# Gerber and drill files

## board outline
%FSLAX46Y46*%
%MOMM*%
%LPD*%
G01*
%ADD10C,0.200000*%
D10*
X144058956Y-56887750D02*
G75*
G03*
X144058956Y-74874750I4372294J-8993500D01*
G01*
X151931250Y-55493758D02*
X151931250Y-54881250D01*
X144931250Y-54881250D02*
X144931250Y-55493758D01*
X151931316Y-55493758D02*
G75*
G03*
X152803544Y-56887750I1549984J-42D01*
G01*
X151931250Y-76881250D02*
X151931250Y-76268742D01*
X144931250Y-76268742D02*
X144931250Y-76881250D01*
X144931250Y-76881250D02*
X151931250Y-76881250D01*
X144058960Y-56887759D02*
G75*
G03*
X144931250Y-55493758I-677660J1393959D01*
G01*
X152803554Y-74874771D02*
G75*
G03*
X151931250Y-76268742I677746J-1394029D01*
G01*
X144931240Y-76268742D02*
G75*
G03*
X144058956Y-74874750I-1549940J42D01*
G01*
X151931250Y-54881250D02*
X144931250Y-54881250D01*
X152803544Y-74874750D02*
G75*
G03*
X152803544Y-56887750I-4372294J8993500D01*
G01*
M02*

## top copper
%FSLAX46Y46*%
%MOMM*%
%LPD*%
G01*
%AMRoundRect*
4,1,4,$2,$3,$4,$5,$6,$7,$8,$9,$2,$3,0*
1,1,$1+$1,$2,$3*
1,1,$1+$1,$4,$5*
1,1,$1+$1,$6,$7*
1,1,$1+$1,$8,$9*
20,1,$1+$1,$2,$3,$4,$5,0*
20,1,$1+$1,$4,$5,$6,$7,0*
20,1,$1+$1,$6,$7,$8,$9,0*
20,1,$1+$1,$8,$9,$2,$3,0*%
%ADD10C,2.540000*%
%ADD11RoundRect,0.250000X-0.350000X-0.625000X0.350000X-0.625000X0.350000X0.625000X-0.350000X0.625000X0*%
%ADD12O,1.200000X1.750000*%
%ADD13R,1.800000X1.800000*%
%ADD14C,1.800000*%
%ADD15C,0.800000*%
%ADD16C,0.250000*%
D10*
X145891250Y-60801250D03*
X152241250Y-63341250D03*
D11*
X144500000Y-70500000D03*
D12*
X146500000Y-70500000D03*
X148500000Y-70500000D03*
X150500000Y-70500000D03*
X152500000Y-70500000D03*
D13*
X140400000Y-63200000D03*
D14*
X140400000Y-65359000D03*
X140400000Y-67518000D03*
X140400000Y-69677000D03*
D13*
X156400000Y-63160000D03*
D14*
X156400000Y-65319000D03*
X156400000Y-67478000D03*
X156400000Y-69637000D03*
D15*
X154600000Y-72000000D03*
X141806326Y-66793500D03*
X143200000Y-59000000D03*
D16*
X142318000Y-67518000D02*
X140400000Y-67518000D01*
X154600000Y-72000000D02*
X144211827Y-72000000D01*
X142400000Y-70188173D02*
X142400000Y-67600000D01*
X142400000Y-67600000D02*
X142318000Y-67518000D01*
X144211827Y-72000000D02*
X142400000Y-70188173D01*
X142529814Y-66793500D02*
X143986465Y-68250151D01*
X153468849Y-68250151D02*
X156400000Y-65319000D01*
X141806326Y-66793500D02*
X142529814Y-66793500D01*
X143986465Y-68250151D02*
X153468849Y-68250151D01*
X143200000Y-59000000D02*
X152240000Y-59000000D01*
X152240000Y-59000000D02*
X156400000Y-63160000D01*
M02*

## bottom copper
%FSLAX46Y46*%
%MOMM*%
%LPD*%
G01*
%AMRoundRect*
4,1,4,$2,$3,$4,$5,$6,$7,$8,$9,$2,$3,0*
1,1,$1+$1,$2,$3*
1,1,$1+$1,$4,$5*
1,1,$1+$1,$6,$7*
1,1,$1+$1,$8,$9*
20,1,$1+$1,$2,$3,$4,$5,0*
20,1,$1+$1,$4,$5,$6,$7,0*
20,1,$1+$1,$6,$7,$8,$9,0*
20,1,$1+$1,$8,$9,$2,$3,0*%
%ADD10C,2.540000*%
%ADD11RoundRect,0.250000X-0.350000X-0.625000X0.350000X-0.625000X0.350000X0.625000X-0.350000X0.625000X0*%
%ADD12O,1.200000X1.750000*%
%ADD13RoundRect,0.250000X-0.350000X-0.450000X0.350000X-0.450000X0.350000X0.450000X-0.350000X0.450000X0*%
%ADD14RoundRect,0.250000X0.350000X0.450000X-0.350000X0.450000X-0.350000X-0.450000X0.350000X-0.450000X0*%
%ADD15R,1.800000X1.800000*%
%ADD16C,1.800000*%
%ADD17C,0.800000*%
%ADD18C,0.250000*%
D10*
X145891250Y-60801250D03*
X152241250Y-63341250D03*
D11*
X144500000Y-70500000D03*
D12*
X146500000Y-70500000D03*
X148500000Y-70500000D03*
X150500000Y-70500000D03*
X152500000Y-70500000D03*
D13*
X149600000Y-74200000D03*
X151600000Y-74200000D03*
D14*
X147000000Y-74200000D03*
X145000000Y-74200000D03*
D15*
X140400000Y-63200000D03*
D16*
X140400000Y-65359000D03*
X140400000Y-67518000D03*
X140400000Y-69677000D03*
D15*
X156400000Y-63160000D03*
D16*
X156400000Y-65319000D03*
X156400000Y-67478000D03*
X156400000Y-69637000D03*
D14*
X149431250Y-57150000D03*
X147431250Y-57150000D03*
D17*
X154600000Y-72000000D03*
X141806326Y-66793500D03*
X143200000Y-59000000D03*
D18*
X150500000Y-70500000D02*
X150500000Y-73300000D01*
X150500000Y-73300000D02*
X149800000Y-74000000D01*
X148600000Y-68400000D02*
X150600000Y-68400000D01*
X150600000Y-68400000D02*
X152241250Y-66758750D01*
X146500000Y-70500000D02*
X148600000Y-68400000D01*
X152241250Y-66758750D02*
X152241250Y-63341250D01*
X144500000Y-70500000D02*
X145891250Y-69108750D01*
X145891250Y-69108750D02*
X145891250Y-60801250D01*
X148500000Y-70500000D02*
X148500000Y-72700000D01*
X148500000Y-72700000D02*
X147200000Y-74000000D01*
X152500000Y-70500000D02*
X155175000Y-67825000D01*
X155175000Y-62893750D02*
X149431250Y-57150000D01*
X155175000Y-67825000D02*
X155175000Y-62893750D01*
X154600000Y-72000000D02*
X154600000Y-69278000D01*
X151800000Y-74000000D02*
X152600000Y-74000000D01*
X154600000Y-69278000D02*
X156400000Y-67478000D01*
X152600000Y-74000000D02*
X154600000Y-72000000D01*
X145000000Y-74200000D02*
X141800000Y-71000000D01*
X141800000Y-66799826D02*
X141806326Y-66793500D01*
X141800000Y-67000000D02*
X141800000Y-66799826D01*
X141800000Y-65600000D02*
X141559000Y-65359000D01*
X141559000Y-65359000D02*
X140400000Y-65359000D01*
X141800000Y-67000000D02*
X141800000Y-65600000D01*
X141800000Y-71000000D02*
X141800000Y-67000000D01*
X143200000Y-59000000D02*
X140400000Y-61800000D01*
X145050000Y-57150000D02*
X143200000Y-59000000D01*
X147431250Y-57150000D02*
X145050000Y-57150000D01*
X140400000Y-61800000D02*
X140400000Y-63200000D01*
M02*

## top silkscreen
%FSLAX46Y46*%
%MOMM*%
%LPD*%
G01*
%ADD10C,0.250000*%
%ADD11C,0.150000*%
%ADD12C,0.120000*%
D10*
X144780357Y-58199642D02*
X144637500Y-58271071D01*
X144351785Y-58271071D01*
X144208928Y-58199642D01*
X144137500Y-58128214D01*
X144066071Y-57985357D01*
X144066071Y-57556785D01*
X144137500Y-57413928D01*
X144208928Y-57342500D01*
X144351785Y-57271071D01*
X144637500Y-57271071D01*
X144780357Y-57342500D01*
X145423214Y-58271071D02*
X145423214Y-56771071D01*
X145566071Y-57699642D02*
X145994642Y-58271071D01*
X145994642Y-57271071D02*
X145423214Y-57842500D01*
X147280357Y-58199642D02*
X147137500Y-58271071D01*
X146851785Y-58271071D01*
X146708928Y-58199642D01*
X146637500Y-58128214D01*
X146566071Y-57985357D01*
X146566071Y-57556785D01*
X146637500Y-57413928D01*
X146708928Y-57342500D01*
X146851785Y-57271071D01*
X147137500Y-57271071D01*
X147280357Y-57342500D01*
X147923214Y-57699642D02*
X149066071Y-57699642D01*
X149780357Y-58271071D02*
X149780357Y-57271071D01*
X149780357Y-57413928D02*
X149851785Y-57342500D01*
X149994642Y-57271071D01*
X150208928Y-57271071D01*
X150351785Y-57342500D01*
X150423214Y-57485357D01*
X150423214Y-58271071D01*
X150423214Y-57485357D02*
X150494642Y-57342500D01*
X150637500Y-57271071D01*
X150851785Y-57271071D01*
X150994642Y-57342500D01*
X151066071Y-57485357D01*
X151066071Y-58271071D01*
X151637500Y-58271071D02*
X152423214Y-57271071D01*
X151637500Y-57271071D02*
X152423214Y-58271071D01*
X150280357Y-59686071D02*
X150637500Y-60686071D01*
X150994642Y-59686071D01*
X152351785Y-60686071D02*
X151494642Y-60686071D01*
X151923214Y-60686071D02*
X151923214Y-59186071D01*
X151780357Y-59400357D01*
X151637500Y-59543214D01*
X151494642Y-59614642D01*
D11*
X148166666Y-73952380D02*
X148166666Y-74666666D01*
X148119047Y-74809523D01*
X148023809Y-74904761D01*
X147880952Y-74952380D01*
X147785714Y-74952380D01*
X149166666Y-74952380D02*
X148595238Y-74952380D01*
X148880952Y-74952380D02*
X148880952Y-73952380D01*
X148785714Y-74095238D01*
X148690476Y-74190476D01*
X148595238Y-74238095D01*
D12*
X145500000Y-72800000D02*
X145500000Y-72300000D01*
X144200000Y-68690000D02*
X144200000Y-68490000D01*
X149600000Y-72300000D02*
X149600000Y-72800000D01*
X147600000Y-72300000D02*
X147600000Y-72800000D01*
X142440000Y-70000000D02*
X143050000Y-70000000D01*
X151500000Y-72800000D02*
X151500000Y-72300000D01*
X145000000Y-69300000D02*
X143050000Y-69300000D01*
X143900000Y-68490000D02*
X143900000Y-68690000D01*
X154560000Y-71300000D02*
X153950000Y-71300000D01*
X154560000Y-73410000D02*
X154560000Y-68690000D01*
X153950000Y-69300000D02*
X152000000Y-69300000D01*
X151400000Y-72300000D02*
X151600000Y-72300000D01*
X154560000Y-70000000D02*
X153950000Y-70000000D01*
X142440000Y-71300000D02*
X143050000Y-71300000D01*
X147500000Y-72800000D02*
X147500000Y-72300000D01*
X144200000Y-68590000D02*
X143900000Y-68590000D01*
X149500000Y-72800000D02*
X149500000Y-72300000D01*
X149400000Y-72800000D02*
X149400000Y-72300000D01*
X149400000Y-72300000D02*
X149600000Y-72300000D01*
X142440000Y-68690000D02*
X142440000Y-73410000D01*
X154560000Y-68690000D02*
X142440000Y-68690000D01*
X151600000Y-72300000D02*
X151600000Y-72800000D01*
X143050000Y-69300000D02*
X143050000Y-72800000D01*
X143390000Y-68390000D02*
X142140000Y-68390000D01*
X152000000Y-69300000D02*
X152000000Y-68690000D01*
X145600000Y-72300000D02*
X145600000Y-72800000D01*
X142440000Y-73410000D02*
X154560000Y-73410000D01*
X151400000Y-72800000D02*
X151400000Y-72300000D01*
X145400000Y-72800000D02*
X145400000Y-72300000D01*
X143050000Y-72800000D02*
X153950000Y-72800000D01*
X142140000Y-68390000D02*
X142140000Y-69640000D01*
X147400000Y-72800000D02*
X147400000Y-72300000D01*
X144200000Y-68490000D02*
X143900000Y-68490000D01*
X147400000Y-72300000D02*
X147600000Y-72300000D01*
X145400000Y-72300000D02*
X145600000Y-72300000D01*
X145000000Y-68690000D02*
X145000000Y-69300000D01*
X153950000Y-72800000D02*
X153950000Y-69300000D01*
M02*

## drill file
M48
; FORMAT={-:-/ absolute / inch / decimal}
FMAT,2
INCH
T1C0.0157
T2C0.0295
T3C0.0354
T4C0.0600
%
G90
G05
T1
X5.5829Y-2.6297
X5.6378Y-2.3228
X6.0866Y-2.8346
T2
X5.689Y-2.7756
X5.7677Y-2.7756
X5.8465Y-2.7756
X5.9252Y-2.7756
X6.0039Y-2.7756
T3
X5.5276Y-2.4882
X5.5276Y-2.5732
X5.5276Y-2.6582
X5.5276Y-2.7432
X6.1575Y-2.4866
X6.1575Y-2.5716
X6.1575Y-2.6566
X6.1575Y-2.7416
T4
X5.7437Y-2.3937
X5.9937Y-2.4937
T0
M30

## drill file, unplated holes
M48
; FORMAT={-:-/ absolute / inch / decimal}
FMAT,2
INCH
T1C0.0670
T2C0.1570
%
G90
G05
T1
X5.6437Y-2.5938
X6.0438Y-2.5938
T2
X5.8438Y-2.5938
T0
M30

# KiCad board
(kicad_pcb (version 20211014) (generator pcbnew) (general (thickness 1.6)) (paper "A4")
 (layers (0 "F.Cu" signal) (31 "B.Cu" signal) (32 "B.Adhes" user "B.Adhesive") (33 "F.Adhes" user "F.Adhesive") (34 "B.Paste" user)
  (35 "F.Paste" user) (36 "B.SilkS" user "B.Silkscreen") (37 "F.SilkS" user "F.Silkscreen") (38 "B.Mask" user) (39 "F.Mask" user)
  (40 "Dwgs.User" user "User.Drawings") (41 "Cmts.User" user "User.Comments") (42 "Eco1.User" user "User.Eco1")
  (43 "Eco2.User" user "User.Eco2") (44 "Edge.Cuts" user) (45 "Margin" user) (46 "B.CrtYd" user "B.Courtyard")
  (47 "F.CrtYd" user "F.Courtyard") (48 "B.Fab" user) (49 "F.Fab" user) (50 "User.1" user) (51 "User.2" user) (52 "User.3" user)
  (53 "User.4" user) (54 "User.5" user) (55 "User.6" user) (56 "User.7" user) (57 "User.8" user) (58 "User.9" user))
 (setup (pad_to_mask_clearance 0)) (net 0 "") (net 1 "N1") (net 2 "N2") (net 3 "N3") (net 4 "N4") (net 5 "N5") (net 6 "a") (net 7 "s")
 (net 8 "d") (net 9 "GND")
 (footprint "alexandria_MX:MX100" (layer "F.Cu") (at 148.43125 65.88125)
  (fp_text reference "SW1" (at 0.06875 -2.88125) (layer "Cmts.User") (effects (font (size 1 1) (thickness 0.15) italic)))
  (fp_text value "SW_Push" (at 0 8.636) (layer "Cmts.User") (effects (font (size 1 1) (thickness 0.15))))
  (pad "" np_thru_hole circle locked (at 5.08 0) (size 1.7018 1.7018) (drill 1.7018) (layers *.Cu *.Mask))
  (pad "" connect circle locked (at -2.54 -5.08) (size 1.524 1.524) (layers "B.Mask"))
  (pad "" np_thru_hole circle locked (at -5.08 0) (size 1.7018 1.7018) (drill 1.7018) (layers *.Cu *.Mask))
  (pad "" connect circle locked (at 3.81 -2.54) (size 1.524 1.524) (layers "B.Mask"))
  (pad "" np_thru_hole circle locked (at 0 0) (size 3.9878 3.9878) (drill 3.9878) (layers *.Cu *.Mask))
  (pad "1" thru_hole circle locked (at -2.54 -5.08) (size 2.54 2.54) (drill 1.524) (layers *.Cu "F.Mask") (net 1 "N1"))
  (pad "2" thru_hole circle locked (at 3.81 -2.54 90) (size 2.54 2.54) (drill 1.524) (layers *.Cu "F.Mask") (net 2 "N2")))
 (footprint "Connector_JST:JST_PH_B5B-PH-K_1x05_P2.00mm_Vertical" (layer "F.Cu") (at 144.5 70.5)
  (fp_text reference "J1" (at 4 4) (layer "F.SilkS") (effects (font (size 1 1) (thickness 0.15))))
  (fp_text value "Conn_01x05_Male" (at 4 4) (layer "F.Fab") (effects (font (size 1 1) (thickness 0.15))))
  (fp_line (start 1 2.3) (end 1 1.8) (layer "F.SilkS") (width 0.12))
  (fp_line (start -0.3 -1.81) (end -0.3 -2.01) (layer "F.SilkS") (width 0.12))
  (fp_line (start 5.1 1.8) (end 5.1 2.3) (layer "F.SilkS") (width 0.12))
  (fp_line (start 3.1 1.8) (end 3.1 2.3) (layer "F.SilkS") (width 0.12))
  (fp_line (start -2.06 -0.5) (end -1.45 -0.5) (layer "F.SilkS") (width 0.12))
  (fp_line (start 7 2.3) (end 7 1.8) (layer "F.SilkS") (width 0.12))
  (fp_line (start 0.5 -1.2) (end -1.45 -1.2) (layer "F.SilkS") (width 0.12))
  (fp_line (start -0.6 -2.01) (end -0.6 -1.81) (layer "F.SilkS") (width 0.12))
  (fp_line (start 10.06 0.8) (end 9.45 0.8) (layer "F.SilkS") (width 0.12))
  (fp_line (start 10.06 2.91) (end 10.06 -1.81) (layer "F.SilkS") (width 0.12))
  (fp_line (start 9.45 -1.2) (end 7.5 -1.2) (layer "F.SilkS") (width 0.12))
  (fp_line (start 6.9 1.8) (end 7.1 1.8) (layer "F.SilkS") (width 0.12))
  (fp_line (start 10.06 -0.5) (end 9.45 -0.5) (layer "F.SilkS") (width 0.12))
  (fp_line (start -2.06 0.8) (end -1.45 0.8) (layer "F.SilkS") (width 0.12))
  (fp_line (start 3 2.3) (end 3 1.8) (layer "F.SilkS") (width 0.12))
  (fp_line (start -0.3 -1.91) (end -0.6 -1.91) (layer "F.SilkS") (width 0.12))
  (fp_line (start 5 2.3) (end 5 1.8) (layer "F.SilkS") (width 0.12))
  (fp_line (start 4.9 2.3) (end 4.9 1.8) (layer "F.SilkS") (width 0.12))
  (fp_line (start 4.9 1.8) (end 5.1 1.8) (layer "F.SilkS") (width 0.12))
  (fp_line (start -2.06 -1.81) (end -2.06 2.91) (layer "F.SilkS") (width 0.12))
  (fp_line (start 10.06 -1.81) (end -2.06 -1.81) (layer "F.SilkS") (width 0.12))
  (fp_line (start 7.1 1.8) (end 7.1 2.3) (layer "F.SilkS") (width 0.12))
  (fp_line (start -1.45 -1.2) (end -1.45 2.3) (layer "F.SilkS") (width 0.12))
  (fp_line (start -1.11 -2.11) (end -2.36 -2.11) (layer "F.SilkS") (width 0.12))
  (fp_line (start 7.5 -1.2) (end 7.5 -1.81) (layer "F.SilkS") (width 0.12))
  (fp_line (start 1.1 1.8) (end 1.1 2.3) (layer "F.SilkS") (width 0.12))
  (fp_line (start -2.06 2.91) (end 10.06 2.91) (layer "F.SilkS") (width 0.12))
  (fp_line (start 6.9 2.3) (end 6.9 1.8) (layer "F.SilkS") (width 0.12))
  (fp_line (start 0.9 2.3) (end 0.9 1.8) (layer "F.SilkS") (width 0.12))
  (fp_line (start -1.45 2.3) (end 9.45 2.3) (layer "F.SilkS") (width 0.12))
  (fp_line (start -2.36 -2.11) (end -2.36 -0.86) (layer "F.SilkS") (width 0.12))
  (fp_line (start 2.9 2.3) (end 2.9 1.8) (layer "F.SilkS") (width 0.12))
  (fp_line (start -0.3 -2.01) (end -0.6 -2.01) (layer "F.SilkS") (width 0.12))
  (fp_line (start 2.9 1.8) (end 3.1 1.8) (layer "F.SilkS") (width 0.12))
  (fp_line (start 0.9 1.8) (end 1.1 1.8) (layer "F.SilkS") (width 0.12))
  (fp_line (start 0.5 -1.81) (end 0.5 -1.2) (layer "F.SilkS") (width 0.12))
  (fp_line (start 9.45 2.3) (end 9.45 -1.2) (layer "F.SilkS") (width 0.12))
  (pad "1" thru_hole roundrect (at 0 0) (size 1.2 1.75) (drill 0.75) (layers *.Cu *.Mask) (roundrect_rratio 0.2083333333) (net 1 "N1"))
  (pad "2" thru_hole oval (at 2 0) (size 1.2 1.75) (drill 0.75) (layers *.Cu *.Mask) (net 2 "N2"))
  (pad "3" thru_hole oval (at 4 0) (size 1.2 1.75) (drill 0.75) (layers *.Cu *.Mask) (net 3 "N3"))
  (pad "4" thru_hole oval (at 6 0) (size 1.2 1.75) (drill 0.75) (layers *.Cu *.Mask) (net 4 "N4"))
  (pad "5" thru_hole oval (at 8 0) (size 1.2 1.75) (drill 0.75) (layers *.Cu *.Mask) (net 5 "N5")))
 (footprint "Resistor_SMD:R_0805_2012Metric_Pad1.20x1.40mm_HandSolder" (layer "B.Cu") (at 150.6 74.2)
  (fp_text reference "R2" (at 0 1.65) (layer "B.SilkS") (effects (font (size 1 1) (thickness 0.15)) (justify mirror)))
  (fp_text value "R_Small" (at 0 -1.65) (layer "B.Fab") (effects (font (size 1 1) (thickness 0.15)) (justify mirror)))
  (pad "1" smd roundrect (at -1 0) (size 1.2 1.4) (layers "B.Cu" "B.Paste" "B.Mask") (roundrect_rratio 0.2083333333) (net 4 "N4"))
  (pad "2" smd roundrect (at 1 0) (size 1.2 1.4) (layers "B.Cu" "B.Paste" "B.Mask") (roundrect_rratio 0.2083333333) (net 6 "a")))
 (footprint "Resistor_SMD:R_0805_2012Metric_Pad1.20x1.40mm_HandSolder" (layer "B.Cu") (at 146 74.2 180)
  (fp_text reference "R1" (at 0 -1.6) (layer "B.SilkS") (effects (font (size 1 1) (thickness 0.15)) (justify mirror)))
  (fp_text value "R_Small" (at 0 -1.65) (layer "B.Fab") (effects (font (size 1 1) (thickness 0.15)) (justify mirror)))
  (pad "1" smd roundrect (at -1 0 180) (size 1.2 1.4) (layers "B.Cu" "B.Paste" "B.Mask") (roundrect_rratio 0.2083333333) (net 3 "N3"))
  (pad "2" smd roundrect (at 1 0 180) (size 1.2 1.4) (layers "B.Cu" "B.Paste" "B.Mask") (roundrect_rratio 0.2083333333) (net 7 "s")))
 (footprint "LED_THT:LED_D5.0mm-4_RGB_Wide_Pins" (layer "B.Cu") (at 140.4 63.2 -90)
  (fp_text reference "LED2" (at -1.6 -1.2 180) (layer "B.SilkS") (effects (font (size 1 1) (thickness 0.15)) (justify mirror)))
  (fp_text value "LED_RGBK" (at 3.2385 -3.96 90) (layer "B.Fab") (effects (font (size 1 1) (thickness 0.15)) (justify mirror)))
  (pad "1" thru_hole rect (at 0 0 270) (size 1.8 1.8) (drill 0.9) (layers *.Cu *.Mask) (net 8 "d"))
  (pad "2" thru_hole circle (at 2.159 0 270) (size 1.8 1.8) (drill 0.9) (layers *.Cu *.Mask) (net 7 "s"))
  (pad "3" thru_hole circle (at 4.318 0 270) (size 1.8 1.8) (drill 0.9) (layers *.Cu *.Mask) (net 6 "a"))
  (pad "4" thru_hole circle (at 6.477 0 270) (size 1.8 1.8) (drill 0.9) (layers *.Cu *.Mask) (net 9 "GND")))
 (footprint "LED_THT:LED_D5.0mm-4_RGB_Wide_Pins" (layer "B.Cu") (at 156.4 63.16 -90)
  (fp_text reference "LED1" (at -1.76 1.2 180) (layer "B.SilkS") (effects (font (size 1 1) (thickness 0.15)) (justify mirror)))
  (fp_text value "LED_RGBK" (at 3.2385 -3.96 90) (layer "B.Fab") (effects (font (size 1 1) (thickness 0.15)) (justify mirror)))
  (pad "1" thru_hole rect (at 0 0 270) (size 1.8 1.8) (drill 0.9) (layers *.Cu *.Mask) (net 8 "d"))
  (pad "2" thru_hole circle (at 2.159 0 270) (size 1.8 1.8) (drill 0.9) (layers *.Cu *.Mask) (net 7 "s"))
  (pad "3" thru_hole circle (at 4.318 0 270) (size 1.8 1.8) (drill 0.9) (layers *.Cu *.Mask) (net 6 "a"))
  (pad "4" thru_hole circle (at 6.477 0 270) (size 1.8 1.8) (drill 0.9) (layers *.Cu *.Mask) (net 9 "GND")))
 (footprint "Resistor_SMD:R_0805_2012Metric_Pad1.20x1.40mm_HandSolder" (layer "B.Cu") (at 148.43125 57.15 180)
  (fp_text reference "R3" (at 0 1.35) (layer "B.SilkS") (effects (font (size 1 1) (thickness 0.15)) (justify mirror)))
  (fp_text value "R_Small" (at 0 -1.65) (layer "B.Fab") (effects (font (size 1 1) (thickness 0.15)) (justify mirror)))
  (pad "1" smd roundrect (at -1 0 180) (size 1.2 1.4) (layers "B.Cu" "B.Paste" "B.Mask") (roundrect_rratio 0.2083333333) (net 5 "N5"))
  (pad "2" smd roundrect (at 1 0 180) (size 1.2 1.4) (layers "B.Cu" "B.Paste" "B.Mask") (roundrect_rratio 0.2083333333) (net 8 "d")))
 (gr_arc locked (start 144.058956 74.87475) (mid 138.43125 65.88125) (end 144.058956 56.88775) (layer "Edge.Cuts") (width 0.2))
 (gr_line locked (start 151.93125 55.493758) (end 151.93125 54.88125) (layer "Edge.Cuts") (width 0.2))
 (gr_line locked (start 144.93125 54.88125) (end 144.93125 55.493758) (layer "Edge.Cuts") (width 0.2))
 (gr_arc locked (start 152.803544 56.88775) (mid 152.167298 56.315967) (end 151.93125 55.493758) (layer "Edge.Cuts") (width 0.2))
 (gr_line locked (start 151.93125 76.88125) (end 151.93125 76.268742) (layer "Edge.Cuts") (width 0.2))
 (gr_line locked (start 144.93125 76.268742) (end 144.93125 76.88125) (layer "Edge.Cuts") (width 0.2))
 (gr_line locked (start 144.93125 76.88125) (end 151.93125 76.88125) (layer "Edge.Cuts") (width 0.2))
 (gr_arc locked (start 144.93125 55.493758) (mid 144.695203 56.315967) (end 144.058956 56.88775) (layer "Edge.Cuts") (width 0.2))
 (gr_arc locked (start 151.93125 76.268742) (mid 152.1673 75.446536) (end 152.803544 74.87475) (layer "Edge.Cuts") (width 0.2))
 (gr_arc locked (start 144.058956 74.87475) (mid 144.695203 75.446533) (end 144.93125 76.268742) (layer "Edge.Cuts") (width 0.2))
 (gr_line locked (start 151.93125 54.88125) (end 144.93125 54.88125) (layer "Edge.Cuts") (width 0.2))
 (gr_arc locked (start 152.803544 56.88775) (mid 158.43125 65.88125) (end 152.803544 74.87475) (layer "Edge.Cuts") (width 0.2))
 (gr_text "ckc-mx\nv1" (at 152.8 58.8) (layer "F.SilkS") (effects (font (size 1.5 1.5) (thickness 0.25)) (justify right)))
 (segment (start 148.6 68.4) (end 150.6 68.4) (width 0.25) (layer "B.Cu") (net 2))
 (segment (start 150.6 68.4) (end 152.24125 66.75875) (width 0.25) (layer "B.Cu") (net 2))
 (segment (start 146.5 70.5) (end 148.6 68.4) (width 0.25) (layer "B.Cu") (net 2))
 (segment (start 152.24125 66.75875) (end 152.24125 63.34125) (width 0.25) (layer "B.Cu") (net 2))
 (segment (start 144.5 70.5) (end 145.89125 69.10875) (width 0.25) (layer "B.Cu") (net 1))
 (segment (start 145.89125 69.10875) (end 145.89125 60.80125) (width 0.25) (layer "B.Cu") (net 1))
 (segment (start 148.5 70.5) (end 148.5 72.7) (width 0.25) (layer "B.Cu") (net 3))
 (segment (start 148.5 72.7) (end 147.2 74) (width 0.25) (layer "B.Cu") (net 3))
 (segment (start 150.5 73.3) (end 149.8 74) (width 0.25) (layer "B.Cu") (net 4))
 (segment (start 150.5 70.5) (end 150.5 73.3) (width 0.25) (layer "B.Cu") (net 4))
 (segment (start 152.5 70.5) (end 155.175 67.825) (width 0.25) (layer "B.Cu") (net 5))
 (segment (start 155.175 62.89375) (end 149.43125 57.15) (width 0.25) (layer "B.Cu") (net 5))
 (segment (start 155.175 67.825) (end 155.175 62.89375) (width 0.25) (layer "B.Cu") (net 5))
 (segment (start 142.318 67.518) (end 140.4 67.518) (width 0.25) (layer "F.Cu") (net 6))
 (segment (start 154.6 72) (end 144.211827 72) (width 0.25) (layer "F.Cu") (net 6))
 (segment (start 142.4 70.188173) (end 142.4 67.6) (width 0.25) (layer "F.Cu") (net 6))
 (segment (start 142.4 67.6) (end 142.318 67.518) (width 0.25) (layer "F.Cu") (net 6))
 (segment (start 144.211827 72) (end 142.4 70.188173) (width 0.25) (layer "F.Cu") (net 6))
 (via (at 154.6 72) (size 0.8) (drill 0.4) (layers "F.Cu" "B.Cu") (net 6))
 (segment (start 154.6 72) (end 154.6 69.278) (width 0.25) (layer "B.Cu") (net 6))
 (segment (start 151.8 74) (end 152.6 74) (width 0.25) (layer "B.Cu") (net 6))
 (segment (start 154.6 69.278) (end 156.4 67.478) (width 0.25) (layer "B.Cu") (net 6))
 (segment (start 152.6 74) (end 154.6 72) (width 0.25) (layer "B.Cu") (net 6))
 (segment (start 142.529814 66.7935) (end 143.986465 68.250151) (width 0.25) (layer "F.Cu") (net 7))
 (segment (start 153.468849 68.250151) (end 156.4 65.319) (width 0.25) (layer "F.Cu") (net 7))
 (segment (start 141.806326 66.7935) (end 142.529814 66.7935) (width 0.25) (layer "F.Cu") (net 7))
 (segment (start 143.986465 68.250151) (end 153.468849 68.250151) (width 0.25) (layer "F.Cu") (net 7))
 (via (at 141.806326 66.7935) (size 0.8) (drill 0.4) (layers "F.Cu" "B.Cu") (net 7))
 (segment (start 145 74.2) (end 141.8 71) (width 0.25) (layer "B.Cu") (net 7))
 (segment (start 141.8 66.799826) (end 141.806326 66.7935) (width 0.25) (layer "B.Cu") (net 7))
 (segment (start 141.8 67) (end 141.8 66.799826) (width 0.25) (layer "B.Cu") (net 7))
 (segment (start 141.8 65.6) (end 141.559 65.359) (width 0.25) (layer "B.Cu") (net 7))
 (segment (start 141.559 65.359) (end 140.4 65.359) (width 0.25) (layer "B.Cu") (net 7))
 (segment (start 141.8 67) (end 141.8 65.6) (width 0.25) (layer "B.Cu") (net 7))
 (segment (start 141.8 71) (end 141.8 67) (width 0.25) (layer "B.Cu") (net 7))
 (segment (start 143.2 59) (end 152.24 59) (width 0.25) (layer "F.Cu") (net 8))
 (segment (start 152.24 59) (end 156.4 63.16) (width 0.25) (layer "F.Cu") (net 8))
 (via (at 143.2 59) (size 0.8) (drill 0.4) (layers "F.Cu" "B.Cu") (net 8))
 (segment (start 143.2 59) (end 140.4 61.8) (width 0.25) (layer "B.Cu") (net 8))
 (segment (start 145.05 57.15) (end 143.2 59) (width 0.25) (layer "B.Cu") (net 8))
 (segment (start 147.43125 57.15) (end 145.05 57.15) (width 0.25) (layer "B.Cu") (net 8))
 (segment (start 140.4 61.8) (end 140.4 63.2) (width 0.25) (layer "B.Cu") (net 8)))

